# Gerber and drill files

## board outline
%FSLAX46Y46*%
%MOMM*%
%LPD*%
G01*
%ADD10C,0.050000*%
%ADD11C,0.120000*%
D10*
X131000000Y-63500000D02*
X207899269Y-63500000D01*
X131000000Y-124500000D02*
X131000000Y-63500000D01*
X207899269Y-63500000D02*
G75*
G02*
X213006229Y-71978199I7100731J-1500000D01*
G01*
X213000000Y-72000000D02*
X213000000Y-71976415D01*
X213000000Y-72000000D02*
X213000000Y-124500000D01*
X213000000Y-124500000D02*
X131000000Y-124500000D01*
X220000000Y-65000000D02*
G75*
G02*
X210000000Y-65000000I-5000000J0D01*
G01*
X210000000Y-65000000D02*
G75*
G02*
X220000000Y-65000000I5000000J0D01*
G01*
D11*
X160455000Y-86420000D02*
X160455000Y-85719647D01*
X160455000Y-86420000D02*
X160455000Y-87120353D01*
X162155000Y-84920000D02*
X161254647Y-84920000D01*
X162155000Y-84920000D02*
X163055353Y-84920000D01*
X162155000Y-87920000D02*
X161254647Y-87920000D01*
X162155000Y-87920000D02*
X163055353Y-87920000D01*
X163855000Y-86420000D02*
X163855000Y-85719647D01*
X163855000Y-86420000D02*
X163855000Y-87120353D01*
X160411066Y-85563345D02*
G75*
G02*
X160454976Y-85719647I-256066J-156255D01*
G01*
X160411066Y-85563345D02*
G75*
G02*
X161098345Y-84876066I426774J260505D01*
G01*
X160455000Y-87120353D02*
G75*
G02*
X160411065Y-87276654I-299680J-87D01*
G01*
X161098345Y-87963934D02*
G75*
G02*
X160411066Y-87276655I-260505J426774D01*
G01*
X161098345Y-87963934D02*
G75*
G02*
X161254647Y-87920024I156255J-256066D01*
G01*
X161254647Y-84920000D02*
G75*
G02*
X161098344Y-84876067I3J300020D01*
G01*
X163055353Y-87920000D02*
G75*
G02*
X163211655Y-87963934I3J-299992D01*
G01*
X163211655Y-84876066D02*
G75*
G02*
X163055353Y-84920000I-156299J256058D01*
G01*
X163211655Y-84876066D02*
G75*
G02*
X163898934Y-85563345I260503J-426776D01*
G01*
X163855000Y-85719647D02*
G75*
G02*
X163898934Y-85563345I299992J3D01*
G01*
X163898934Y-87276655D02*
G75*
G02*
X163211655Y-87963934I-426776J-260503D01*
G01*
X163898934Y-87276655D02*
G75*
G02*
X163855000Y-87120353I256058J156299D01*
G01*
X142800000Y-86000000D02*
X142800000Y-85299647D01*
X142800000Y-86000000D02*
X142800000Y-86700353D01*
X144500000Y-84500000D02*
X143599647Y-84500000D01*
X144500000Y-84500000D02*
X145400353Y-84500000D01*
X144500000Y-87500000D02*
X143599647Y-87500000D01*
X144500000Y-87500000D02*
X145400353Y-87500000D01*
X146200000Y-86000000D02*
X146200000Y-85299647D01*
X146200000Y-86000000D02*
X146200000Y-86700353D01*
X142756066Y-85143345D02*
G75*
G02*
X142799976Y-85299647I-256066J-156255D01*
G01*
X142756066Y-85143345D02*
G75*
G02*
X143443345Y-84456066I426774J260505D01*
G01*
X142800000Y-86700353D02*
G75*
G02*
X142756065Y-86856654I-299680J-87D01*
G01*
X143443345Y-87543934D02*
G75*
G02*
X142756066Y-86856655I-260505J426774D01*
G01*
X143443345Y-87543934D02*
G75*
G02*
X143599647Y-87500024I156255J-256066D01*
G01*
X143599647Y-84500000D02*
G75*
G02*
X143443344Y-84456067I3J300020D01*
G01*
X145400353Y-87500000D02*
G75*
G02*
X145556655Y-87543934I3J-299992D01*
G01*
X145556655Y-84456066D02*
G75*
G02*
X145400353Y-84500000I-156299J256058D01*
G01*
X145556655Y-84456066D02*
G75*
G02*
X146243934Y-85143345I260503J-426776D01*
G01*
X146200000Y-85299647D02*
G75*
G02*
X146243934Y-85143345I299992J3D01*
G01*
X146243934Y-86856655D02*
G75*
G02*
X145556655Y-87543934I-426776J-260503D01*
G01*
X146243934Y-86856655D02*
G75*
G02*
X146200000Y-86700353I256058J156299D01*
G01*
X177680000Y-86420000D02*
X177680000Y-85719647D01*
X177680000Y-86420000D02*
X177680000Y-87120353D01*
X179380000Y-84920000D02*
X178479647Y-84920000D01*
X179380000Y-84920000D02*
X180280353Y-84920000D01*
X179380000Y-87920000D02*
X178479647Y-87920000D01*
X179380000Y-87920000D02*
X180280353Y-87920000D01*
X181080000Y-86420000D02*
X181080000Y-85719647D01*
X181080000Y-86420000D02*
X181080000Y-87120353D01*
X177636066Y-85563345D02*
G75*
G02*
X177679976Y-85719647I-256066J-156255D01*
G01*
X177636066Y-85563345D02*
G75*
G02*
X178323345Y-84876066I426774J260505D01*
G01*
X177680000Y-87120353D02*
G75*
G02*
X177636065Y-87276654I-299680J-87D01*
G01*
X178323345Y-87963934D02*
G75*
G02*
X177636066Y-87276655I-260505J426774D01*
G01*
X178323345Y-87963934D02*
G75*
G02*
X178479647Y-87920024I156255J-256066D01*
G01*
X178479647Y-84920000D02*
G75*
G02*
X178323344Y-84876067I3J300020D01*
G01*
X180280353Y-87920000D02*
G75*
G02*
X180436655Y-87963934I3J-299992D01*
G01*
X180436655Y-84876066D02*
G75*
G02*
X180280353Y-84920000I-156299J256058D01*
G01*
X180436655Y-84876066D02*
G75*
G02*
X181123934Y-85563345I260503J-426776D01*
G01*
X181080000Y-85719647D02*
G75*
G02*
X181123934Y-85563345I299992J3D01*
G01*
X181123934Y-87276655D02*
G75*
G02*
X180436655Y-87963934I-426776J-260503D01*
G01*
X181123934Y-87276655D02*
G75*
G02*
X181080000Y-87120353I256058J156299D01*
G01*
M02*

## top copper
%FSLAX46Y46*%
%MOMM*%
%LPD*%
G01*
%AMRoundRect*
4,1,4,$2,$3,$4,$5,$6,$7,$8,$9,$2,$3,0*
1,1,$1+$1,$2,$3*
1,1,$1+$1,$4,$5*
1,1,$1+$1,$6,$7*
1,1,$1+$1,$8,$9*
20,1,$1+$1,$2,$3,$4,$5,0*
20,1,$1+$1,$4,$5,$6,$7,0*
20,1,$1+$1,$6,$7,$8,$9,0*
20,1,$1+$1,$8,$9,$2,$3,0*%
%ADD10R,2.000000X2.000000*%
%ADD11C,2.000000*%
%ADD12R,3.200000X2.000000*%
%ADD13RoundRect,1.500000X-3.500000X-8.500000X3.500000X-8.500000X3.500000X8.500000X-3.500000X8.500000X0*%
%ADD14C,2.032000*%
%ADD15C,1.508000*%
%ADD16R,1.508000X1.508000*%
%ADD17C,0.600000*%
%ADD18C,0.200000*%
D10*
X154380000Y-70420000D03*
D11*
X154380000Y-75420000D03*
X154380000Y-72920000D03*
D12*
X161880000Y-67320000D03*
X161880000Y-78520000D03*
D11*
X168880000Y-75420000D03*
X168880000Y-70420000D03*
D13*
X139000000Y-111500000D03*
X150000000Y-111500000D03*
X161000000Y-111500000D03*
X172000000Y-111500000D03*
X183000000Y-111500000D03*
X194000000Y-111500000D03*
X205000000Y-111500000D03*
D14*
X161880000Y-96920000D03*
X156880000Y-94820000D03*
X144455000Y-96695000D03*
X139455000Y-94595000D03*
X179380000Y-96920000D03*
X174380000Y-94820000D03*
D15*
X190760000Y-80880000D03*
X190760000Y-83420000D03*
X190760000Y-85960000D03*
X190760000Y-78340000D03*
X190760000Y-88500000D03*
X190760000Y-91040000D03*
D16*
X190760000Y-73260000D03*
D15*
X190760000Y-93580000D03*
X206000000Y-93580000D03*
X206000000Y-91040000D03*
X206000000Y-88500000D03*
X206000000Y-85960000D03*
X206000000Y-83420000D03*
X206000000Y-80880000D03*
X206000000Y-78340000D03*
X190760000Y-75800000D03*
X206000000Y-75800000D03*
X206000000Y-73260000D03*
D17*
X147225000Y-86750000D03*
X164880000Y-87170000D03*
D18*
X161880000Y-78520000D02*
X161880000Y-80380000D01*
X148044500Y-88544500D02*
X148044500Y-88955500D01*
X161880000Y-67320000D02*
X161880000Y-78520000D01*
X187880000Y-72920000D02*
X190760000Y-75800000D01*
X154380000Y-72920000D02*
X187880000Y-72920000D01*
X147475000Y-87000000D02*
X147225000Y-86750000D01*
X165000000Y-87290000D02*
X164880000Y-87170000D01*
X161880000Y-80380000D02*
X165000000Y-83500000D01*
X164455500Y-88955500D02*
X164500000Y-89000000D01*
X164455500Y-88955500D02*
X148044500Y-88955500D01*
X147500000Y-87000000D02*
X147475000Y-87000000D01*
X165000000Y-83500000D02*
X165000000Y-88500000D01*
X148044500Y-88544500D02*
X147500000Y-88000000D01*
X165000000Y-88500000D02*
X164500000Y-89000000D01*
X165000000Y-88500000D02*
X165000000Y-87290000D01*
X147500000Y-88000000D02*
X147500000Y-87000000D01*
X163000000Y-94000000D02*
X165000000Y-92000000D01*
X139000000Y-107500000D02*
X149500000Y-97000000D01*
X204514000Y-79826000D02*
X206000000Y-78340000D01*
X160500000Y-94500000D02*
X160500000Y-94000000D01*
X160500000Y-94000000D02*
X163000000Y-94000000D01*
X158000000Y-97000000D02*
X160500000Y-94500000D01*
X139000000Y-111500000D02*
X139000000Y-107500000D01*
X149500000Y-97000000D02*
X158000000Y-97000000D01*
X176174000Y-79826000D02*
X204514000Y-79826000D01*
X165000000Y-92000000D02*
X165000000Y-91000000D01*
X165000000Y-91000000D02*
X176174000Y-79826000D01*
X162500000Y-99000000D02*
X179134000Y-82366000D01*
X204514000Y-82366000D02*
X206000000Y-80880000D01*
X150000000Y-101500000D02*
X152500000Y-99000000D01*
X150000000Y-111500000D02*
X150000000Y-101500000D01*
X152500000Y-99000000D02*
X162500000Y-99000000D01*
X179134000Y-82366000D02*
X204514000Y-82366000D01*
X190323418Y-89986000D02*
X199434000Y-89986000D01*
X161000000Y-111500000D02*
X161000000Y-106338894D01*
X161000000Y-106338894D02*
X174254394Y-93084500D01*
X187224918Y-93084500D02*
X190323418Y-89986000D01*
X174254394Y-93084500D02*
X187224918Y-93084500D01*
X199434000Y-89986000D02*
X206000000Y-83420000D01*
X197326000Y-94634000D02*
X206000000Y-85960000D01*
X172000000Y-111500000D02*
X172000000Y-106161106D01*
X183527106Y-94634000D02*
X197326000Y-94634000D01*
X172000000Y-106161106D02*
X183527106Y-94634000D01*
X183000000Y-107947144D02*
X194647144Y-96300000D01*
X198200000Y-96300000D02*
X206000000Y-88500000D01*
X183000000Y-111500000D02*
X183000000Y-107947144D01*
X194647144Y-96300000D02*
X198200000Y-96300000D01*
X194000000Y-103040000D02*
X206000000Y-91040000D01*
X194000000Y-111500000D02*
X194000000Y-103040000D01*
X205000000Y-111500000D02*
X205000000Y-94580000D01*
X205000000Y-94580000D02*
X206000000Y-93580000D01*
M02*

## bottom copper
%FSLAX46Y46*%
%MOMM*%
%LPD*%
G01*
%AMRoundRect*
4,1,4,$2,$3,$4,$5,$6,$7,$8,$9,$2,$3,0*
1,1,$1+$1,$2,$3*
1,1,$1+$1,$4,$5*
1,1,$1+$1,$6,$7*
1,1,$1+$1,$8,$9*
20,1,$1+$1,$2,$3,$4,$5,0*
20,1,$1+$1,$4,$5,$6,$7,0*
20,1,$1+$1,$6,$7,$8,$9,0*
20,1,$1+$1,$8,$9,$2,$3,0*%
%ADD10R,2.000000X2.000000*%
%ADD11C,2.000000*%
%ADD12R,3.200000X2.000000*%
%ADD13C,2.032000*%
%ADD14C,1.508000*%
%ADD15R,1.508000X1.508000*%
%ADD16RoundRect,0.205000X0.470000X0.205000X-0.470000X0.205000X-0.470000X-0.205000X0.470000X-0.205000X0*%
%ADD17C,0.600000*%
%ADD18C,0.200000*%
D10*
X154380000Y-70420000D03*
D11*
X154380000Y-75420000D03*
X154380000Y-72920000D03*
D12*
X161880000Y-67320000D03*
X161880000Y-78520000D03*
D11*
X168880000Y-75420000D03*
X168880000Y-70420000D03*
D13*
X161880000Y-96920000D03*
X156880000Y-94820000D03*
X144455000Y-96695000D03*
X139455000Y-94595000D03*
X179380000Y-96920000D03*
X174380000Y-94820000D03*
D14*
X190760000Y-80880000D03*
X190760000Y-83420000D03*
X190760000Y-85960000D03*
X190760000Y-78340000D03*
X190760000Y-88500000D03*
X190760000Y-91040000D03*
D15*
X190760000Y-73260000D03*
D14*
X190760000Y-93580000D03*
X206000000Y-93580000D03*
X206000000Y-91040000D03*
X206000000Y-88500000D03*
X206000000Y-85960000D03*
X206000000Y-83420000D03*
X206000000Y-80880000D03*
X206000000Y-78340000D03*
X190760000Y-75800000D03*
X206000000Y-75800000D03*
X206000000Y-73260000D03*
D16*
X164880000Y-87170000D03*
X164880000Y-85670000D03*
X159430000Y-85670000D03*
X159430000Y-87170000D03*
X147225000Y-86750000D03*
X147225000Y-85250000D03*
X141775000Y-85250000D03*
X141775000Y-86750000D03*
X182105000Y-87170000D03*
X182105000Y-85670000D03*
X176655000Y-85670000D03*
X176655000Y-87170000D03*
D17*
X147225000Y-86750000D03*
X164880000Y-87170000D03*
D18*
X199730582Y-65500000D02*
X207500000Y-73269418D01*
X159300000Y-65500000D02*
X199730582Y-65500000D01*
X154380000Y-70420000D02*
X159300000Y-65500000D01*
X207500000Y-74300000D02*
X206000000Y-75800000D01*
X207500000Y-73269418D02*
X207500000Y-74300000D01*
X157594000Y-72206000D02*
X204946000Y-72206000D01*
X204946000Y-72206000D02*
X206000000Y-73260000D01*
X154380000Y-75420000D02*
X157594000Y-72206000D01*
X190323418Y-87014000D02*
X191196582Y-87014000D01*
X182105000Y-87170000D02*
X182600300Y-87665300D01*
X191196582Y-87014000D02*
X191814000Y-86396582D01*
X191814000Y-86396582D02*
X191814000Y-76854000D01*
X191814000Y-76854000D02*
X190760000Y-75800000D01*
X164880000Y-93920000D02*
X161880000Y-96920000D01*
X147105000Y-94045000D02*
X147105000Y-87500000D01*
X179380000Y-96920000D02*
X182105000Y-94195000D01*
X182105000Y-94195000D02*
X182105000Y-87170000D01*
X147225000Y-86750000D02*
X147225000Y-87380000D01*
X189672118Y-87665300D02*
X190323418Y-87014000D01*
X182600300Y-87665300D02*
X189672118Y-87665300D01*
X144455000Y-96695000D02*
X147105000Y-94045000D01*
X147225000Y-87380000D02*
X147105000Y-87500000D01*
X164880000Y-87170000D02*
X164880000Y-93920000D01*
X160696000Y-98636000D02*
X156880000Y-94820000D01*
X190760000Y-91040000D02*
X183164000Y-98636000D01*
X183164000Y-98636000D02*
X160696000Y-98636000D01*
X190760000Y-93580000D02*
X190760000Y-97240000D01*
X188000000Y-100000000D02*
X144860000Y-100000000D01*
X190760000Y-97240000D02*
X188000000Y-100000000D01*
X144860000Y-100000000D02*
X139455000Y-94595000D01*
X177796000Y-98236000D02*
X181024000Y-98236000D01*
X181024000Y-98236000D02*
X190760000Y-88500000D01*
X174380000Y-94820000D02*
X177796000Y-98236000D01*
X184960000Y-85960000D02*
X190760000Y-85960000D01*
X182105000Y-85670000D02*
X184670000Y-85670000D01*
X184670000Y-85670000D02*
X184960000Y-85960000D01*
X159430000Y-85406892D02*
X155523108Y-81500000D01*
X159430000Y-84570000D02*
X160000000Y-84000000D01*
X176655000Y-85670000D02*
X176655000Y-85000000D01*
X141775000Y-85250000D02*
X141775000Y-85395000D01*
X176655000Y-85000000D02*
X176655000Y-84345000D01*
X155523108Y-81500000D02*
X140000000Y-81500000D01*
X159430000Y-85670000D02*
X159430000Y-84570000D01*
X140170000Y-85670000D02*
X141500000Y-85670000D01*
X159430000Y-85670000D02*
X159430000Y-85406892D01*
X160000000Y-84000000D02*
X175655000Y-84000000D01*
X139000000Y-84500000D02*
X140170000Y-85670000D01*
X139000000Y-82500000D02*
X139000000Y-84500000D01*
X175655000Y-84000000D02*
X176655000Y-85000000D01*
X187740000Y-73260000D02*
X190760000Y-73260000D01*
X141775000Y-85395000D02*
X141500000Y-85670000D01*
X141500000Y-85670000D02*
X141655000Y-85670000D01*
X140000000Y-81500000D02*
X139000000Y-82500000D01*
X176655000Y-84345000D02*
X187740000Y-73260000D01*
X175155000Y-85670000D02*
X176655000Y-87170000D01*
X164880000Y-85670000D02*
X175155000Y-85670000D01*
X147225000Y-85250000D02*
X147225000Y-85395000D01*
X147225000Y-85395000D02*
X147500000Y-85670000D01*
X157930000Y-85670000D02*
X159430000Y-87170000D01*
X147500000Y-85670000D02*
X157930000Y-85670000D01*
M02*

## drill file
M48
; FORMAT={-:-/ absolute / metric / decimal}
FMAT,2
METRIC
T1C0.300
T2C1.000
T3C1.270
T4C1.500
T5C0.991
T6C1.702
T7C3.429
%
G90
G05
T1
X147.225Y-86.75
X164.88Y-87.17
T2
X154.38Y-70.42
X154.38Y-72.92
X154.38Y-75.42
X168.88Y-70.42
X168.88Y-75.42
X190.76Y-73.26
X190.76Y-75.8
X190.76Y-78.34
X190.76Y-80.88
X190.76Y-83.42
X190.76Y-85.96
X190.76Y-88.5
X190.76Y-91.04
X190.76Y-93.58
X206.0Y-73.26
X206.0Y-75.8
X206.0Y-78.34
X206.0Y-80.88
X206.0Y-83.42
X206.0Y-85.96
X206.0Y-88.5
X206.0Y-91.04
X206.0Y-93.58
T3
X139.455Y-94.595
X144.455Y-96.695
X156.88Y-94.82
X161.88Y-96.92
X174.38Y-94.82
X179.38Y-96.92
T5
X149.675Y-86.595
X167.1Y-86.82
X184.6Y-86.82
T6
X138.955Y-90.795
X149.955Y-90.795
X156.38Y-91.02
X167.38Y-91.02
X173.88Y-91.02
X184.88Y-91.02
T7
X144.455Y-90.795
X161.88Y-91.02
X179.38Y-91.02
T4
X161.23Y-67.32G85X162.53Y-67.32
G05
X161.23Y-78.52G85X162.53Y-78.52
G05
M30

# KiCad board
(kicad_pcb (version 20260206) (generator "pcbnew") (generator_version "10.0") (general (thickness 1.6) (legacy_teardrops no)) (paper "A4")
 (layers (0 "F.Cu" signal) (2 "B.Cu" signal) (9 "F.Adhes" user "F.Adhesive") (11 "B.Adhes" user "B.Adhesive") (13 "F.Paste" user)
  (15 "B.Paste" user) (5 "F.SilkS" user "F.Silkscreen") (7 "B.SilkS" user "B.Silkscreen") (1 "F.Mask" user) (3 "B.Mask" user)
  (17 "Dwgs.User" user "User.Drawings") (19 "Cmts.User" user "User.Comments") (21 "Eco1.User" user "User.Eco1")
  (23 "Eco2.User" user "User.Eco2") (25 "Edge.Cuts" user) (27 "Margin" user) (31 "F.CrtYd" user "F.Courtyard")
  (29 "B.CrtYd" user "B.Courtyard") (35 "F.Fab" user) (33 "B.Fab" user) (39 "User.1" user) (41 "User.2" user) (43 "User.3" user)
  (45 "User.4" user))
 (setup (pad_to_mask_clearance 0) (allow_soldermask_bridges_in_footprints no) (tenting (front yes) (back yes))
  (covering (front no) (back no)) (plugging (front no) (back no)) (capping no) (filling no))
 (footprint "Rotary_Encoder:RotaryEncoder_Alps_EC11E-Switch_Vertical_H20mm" (layer "F.Cu") (at 154.38 70.42)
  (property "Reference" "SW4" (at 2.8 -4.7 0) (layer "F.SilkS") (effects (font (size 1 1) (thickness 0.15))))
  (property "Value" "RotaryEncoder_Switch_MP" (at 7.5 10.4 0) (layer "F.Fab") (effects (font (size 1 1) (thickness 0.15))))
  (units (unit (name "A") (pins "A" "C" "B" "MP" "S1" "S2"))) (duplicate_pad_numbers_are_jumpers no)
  (pad "A" thru_hole rect (at 0 0) (size 2 2) (drill 1) (layers "*.Cu" "*.Mask") (remove_unused_layers no) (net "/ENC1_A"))
  (pad "B" thru_hole circle (at 0 5) (size 2 2) (drill 1) (layers "*.Cu" "*.Mask") (remove_unused_layers no) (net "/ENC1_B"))
  (pad "C" thru_hole circle (at 0 2.5) (size 2 2) (drill 1) (layers "*.Cu" "*.Mask") (remove_unused_layers no) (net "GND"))
  (pad "MP" thru_hole rect (at 7.5 -3.1) (size 3.2 2) (drill oval 2.8 1.5) (layers "*.Cu" "*.Mask") (remove_unused_layers no) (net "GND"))
  (pad "MP" thru_hole rect (at 7.5 8.1) (size 3.2 2) (drill oval 2.8 1.5) (layers "*.Cu" "*.Mask") (remove_unused_layers no) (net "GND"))
  (pad "S1" thru_hole circle (at 14.5 5) (size 2 2) (drill 1) (layers "*.Cu" "*.Mask") (remove_unused_layers no)
   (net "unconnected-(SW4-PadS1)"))
  (pad "S2" thru_hole circle (at 14.5 0) (size 2 2) (drill 1) (layers "*.Cu" "*.Mask") (remove_unused_layers no)
   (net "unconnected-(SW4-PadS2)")))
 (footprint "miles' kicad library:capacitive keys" (layer "F.Cu") (at 169 93.5)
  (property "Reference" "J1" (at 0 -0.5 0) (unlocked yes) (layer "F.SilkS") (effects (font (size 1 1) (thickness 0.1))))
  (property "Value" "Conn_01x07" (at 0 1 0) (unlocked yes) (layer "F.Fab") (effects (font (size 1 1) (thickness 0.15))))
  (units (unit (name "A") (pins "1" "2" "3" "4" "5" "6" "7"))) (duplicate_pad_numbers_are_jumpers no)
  (pad "1" smd roundrect (at -30 18) (size 10 20) (layers "F.Cu" "F.Mask") (roundrect_rratio 0.15) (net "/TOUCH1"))
  (pad "2" smd roundrect (at -19 18) (size 10 20) (layers "F.Cu" "F.Mask") (roundrect_rratio 0.15) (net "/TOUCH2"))
  (pad "3" smd roundrect (at -8 18) (size 10 20) (layers "F.Cu" "F.Mask") (roundrect_rratio 0.15) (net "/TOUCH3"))
  (pad "4" smd roundrect (at 3 18) (size 10 20) (layers "F.Cu" "F.Mask") (roundrect_rratio 0.15) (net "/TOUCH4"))
  (pad "5" smd roundrect (at 14 18) (size 10 20) (layers "F.Cu" "F.Mask") (roundrect_rratio 0.15) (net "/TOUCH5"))
  (pad "6" smd roundrect (at 25 18) (size 10 20) (layers "F.Cu" "F.Mask") (roundrect_rratio 0.15) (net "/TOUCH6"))
  (pad "7" smd roundrect (at 36 18) (size 10 20) (layers "F.Cu" "F.Mask") (roundrect_rratio 0.15) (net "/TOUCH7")))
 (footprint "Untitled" (layer "F.Cu") (at 163 40.5)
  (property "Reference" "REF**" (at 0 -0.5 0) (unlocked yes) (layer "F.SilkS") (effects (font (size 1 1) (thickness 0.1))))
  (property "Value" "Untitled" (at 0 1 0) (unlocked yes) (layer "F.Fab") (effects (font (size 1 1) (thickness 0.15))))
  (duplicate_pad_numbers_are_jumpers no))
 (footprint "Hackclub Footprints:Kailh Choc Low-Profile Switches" (layer "F.Cu") (at 161.88 91.02)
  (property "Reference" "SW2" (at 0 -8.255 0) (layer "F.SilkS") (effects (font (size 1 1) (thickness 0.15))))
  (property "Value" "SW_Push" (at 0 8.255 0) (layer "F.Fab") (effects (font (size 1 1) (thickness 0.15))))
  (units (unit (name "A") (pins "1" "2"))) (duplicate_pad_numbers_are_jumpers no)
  (pad "" np_thru_hole circle (at -5.5 0) (size 1.7018 1.7018) (drill 1.7018) (layers "*.Cu" "*.Mask"))
  (pad "" np_thru_hole circle (at 0 0) (size 3.429 3.429) (drill 3.429) (layers "*.Cu" "*.Mask"))
  (pad "" np_thru_hole circle (at 5.22 -4.2) (size 0.9906 0.9906) (drill 0.9906) (layers "*.Cu" "*.Mask"))
  (pad "" np_thru_hole circle (at 5.5 0) (size 1.7018 1.7018) (drill 1.7018) (layers "*.Cu" "*.Mask"))
  (pad "1" thru_hole circle (at 0 5.9) (size 2.032 2.032) (drill 1.27) (layers "*.Cu" "*.Mask") (remove_unused_layers no) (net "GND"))
  (pad "2" thru_hole circle (at -5 3.8) (size 2.032 2.032) (drill 1.27) (layers "*.Cu" "*.Mask") (remove_unused_layers no) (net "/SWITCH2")))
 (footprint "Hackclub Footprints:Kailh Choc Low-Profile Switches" (layer "F.Cu") (at 144.455 90.795)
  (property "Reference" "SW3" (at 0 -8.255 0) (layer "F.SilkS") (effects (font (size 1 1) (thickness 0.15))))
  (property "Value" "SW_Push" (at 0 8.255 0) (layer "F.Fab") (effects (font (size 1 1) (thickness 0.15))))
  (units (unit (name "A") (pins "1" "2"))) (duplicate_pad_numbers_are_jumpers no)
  (pad "" np_thru_hole circle (at -5.5 0) (size 1.7018 1.7018) (drill 1.7018) (layers "*.Cu" "*.Mask"))
  (pad "" np_thru_hole circle (at 0 0) (size 3.429 3.429) (drill 3.429) (layers "*.Cu" "*.Mask"))
  (pad "" np_thru_hole circle (at 5.22 -4.2) (size 0.9906 0.9906) (drill 0.9906) (layers "*.Cu" "*.Mask"))
  (pad "" np_thru_hole circle (at 5.5 0) (size 1.7018 1.7018) (drill 1.7018) (layers "*.Cu" "*.Mask"))
  (pad "1" thru_hole circle (at 0 5.9) (size 2.032 2.032) (drill 1.27) (layers "*.Cu" "*.Mask") (remove_unused_layers no) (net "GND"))
  (pad "2" thru_hole circle (at -5 3.8) (size 2.032 2.032) (drill 1.27) (layers "*.Cu" "*.Mask") (remove_unused_layers no) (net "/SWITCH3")))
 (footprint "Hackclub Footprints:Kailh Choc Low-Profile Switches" (layer "F.Cu") (at 179.38 91.02)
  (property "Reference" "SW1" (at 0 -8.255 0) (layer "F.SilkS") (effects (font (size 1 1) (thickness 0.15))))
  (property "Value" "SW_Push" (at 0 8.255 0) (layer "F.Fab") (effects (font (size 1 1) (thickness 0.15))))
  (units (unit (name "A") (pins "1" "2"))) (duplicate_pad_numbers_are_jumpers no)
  (pad "" np_thru_hole circle (at -5.5 0) (size 1.7018 1.7018) (drill 1.7018) (layers "*.Cu" "*.Mask"))
  (pad "" np_thru_hole circle (at 0 0) (size 3.429 3.429) (drill 3.429) (layers "*.Cu" "*.Mask"))
  (pad "" np_thru_hole circle (at 5.22 -4.2) (size 0.9906 0.9906) (drill 0.9906) (layers "*.Cu" "*.Mask"))
  (pad "" np_thru_hole circle (at 5.5 0) (size 1.7018 1.7018) (drill 1.7018) (layers "*.Cu" "*.Mask"))
  (pad "1" thru_hole circle (at 0 5.9) (size 2.032 2.032) (drill 1.27) (layers "*.Cu" "*.Mask") (remove_unused_layers no) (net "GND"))
  (pad "2" thru_hole circle (at -5 3.8) (size 2.032 2.032) (drill 1.27) (layers "*.Cu" "*.Mask") (remove_unused_layers no) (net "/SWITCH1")))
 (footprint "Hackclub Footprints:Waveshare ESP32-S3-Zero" (layer "F.Cu") (at 198.38 83.42)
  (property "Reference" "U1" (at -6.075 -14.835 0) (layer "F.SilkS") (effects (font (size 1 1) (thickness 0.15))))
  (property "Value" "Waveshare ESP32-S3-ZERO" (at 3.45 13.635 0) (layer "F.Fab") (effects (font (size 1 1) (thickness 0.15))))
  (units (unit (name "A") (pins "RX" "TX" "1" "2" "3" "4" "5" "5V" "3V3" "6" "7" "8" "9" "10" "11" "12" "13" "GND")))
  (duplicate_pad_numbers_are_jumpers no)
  (pad "1" thru_hole circle (at -7.62 -2.54) (size 1.508 1.508) (drill 1) (layers "*.Cu" "*.Mask") (remove_unused_layers no)
   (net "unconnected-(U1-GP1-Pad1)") (solder_mask_margin 0.102))
  (pad "2" thru_hole circle (at -7.62 0) (size 1.508 1.508) (drill 1) (layers "*.Cu" "*.Mask") (remove_unused_layers no)
   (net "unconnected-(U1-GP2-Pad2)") (solder_mask_margin 0.102))
  (pad "3" thru_hole circle (at -7.62 2.54) (size 1.508 1.508) (drill 1) (layers "*.Cu" "*.Mask") (remove_unused_layers no) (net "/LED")
   (solder_mask_margin 0.102))
  (pad "3V3" thru_hole circle (at -7.62 -5.08) (size 1.508 1.508) (drill 1) (layers "*.Cu" "*.Mask") (remove_unused_layers no) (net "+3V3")
   (solder_mask_margin 0.102))
  (pad "4" thru_hole circle (at -7.62 5.08) (size 1.508 1.508) (drill 1) (layers "*.Cu" "*.Mask") (remove_unused_layers no) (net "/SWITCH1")
   (solder_mask_margin 0.102))
  (pad "5" thru_hole circle (at -7.62 7.62) (size 1.508 1.508) (drill 1) (layers "*.Cu" "*.Mask") (remove_unused_layers no) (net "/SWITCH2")
   (solder_mask_margin 0.102))
  (pad "5V" thru_hole rect (at -7.62 -10.16) (size 1.508 1.508) (drill 1) (layers "*.Cu" "*.Mask") (remove_unused_layers no) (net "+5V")
   (solder_mask_margin 0.102))
  (pad "6" thru_hole circle (at -7.62 10.16) (size 1.508 1.508) (drill 1) (layers "*.Cu" "*.Mask") (remove_unused_layers no)
   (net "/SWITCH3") (solder_mask_margin 0.102))
  (pad "7" thru_hole circle (at 7.62 10.16) (size 1.508 1.508) (drill 1) (layers "*.Cu" "*.Mask") (remove_unused_layers no) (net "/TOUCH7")
   (solder_mask_margin 0.102))
  (pad "8" thru_hole circle (at 7.62 7.62) (size 1.508 1.508) (drill 1) (layers "*.Cu" "*.Mask") (remove_unused_layers no) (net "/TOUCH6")
   (solder_mask_margin 0.102))
  (pad "9" thru_hole circle (at 7.62 5.08) (size 1.508 1.508) (drill 1) (layers "*.Cu" "*.Mask") (remove_unused_layers no) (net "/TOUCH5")
   (solder_mask_margin 0.102))
  (pad "10" thru_hole circle (at 7.62 2.54) (size 1.508 1.508) (drill 1) (layers "*.Cu" "*.Mask") (remove_unused_layers no) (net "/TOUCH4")
   (solder_mask_margin 0.102))
  (pad "11" thru_hole circle (at 7.62 0) (size 1.508 1.508) (drill 1) (layers "*.Cu" "*.Mask") (remove_unused_layers no) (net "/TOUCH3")
   (solder_mask_margin 0.102))
  (pad "12" thru_hole circle (at 7.62 -2.54) (size 1.508 1.508) (drill 1) (layers "*.Cu" "*.Mask") (remove_unused_layers no) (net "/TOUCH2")
   (solder_mask_margin 0.102))
  (pad "13" thru_hole circle (at 7.62 -5.08) (size 1.508 1.508) (drill 1) (layers "*.Cu" "*.Mask") (remove_unused_layers no) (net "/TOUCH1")
   (solder_mask_margin 0.102))
  (pad "GND" thru_hole circle (at -7.62 -7.62) (size 1.508 1.508) (drill 1) (layers "*.Cu" "*.Mask") (remove_unused_layers no) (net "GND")
   (solder_mask_margin 0.102))
  (pad "RX" thru_hole circle (at 7.62 -7.62) (size 1.508 1.508) (drill 1) (layers "*.Cu" "*.Mask") (remove_unused_layers no) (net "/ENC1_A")
   (solder_mask_margin 0.102))
  (pad "TX" thru_hole circle (at 7.62 -10.16) (size 1.508 1.508) (drill 1) (layers "*.Cu" "*.Mask") (remove_unused_layers no)
   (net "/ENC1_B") (solder_mask_margin 0.102)))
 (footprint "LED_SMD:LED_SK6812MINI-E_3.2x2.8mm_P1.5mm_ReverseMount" (layer "B.Cu") (at 162.155 86.42 180)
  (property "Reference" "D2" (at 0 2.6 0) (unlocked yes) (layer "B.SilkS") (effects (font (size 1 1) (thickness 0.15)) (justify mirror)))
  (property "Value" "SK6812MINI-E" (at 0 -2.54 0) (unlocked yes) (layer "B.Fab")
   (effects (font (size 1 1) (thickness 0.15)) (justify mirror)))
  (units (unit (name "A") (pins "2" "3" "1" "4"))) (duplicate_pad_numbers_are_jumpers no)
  (fp_line (start 1.7 0) (end 1.7 0.700353) (stroke (width 0.12) (type solid)) (layer "Edge.Cuts"))
  (fp_line (start 1.7 0) (end 1.7 -0.700353) (stroke (width 0.12) (type solid)) (layer "Edge.Cuts"))
  (fp_line (start 0 1.5) (end 0.900353 1.5) (stroke (width 0.12) (type solid)) (layer "Edge.Cuts"))
  (fp_line (start 0 1.5) (end -0.900353 1.5) (stroke (width 0.12) (type solid)) (layer "Edge.Cuts"))
  (fp_line (start 0 -1.5) (end 0.900353 -1.5) (stroke (width 0.12) (type solid)) (layer "Edge.Cuts"))
  (fp_line (start 0 -1.5) (end -0.900353 -1.5) (stroke (width 0.12) (type solid)) (layer "Edge.Cuts"))
  (fp_line (start -1.7 0) (end -1.7 0.700353) (stroke (width 0.12) (type solid)) (layer "Edge.Cuts"))
  (fp_line (start -1.7 0) (end -1.7 -0.700353) (stroke (width 0.12) (type solid)) (layer "Edge.Cuts"))
  (fp_arc (start 1.743934 0.856655) (mid 1.711191 0.781533) (end 1.7 0.700353) (stroke (width 0.12) (type solid)) (layer "Edge.Cuts"))
  (fp_arc (start 1.743934 0.856655) (mid 1.670713 1.470713) (end 1.056655 1.543934) (stroke (width 0.12) (type solid)) (layer "Edge.Cuts"))
  (fp_arc (start 1.7 -0.700353) (mid 1.711181 -0.781538) (end 1.743934 -0.856655) (stroke (width 0.12) (type solid)) (layer "Edge.Cuts"))
  (fp_arc (start 1.056655 -1.543934) (mid 1.670711 -1.470711) (end 1.743934 -0.856655) (stroke (width 0.12) (type solid))
   (layer "Edge.Cuts"))
  (fp_arc (start 1.056655 -1.543934) (mid 0.981533 -1.511191) (end 0.900353 -1.5) (stroke (width 0.12) (type solid)) (layer "Edge.Cuts"))
  (fp_arc (start 0.900353 1.5) (mid 0.981532 1.511193) (end 1.056655 1.543934) (stroke (width 0.12) (type solid)) (layer "Edge.Cuts"))
  (fp_arc (start -0.900353 -1.5) (mid -0.981533 -1.511192) (end -1.056655 -1.543934) (stroke (width 0.12) (type solid)) (layer "Edge.Cuts"))
  (fp_arc (start -1.056655 1.543934) (mid -0.981533 1.511192) (end -0.900353 1.5) (stroke (width 0.12) (type solid)) (layer "Edge.Cuts"))
  (fp_arc (start -1.056655 1.543934) (mid -1.670711 1.470711) (end -1.743934 0.856655) (stroke (width 0.12) (type solid))
   (layer "Edge.Cuts"))
  (fp_arc (start -1.7 0.700353) (mid -1.711192 0.781533) (end -1.743934 0.856655) (stroke (width 0.12) (type solid)) (layer "Edge.Cuts"))
  (fp_arc (start -1.743934 -0.856655) (mid -1.670711 -1.470711) (end -1.056655 -1.543934) (stroke (width 0.12) (type solid))
   (layer "Edge.Cuts"))
  (fp_arc (start -1.743934 -0.856655) (mid -1.711192 -0.781533) (end -1.7 -0.700353) (stroke (width 0.12) (type solid)) (layer "Edge.Cuts"))
  (pad "1" smd roundrect (at -2.725 -0.75 180) (size 1.35 0.82) (layers "B.Cu" "B.Mask" "B.Paste") (roundrect_rratio 0.25) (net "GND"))
  (pad "2" smd roundrect (at -2.725 0.75 180) (size 1.35 0.82) (layers "B.Cu" "B.Mask" "B.Paste") (roundrect_rratio 0.25)
   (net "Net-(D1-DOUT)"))
  (pad "3" smd roundrect (at 2.725 0.75 180) (size 1.35 0.82) (layers "B.Cu" "B.Mask" "B.Paste") (roundrect_rratio 0.25) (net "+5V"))
  (pad "4" smd roundrect (at 2.725 -0.75 180) (size 1.35 0.82) (layers "B.Cu" "B.Mask" "B.Paste") (roundrect_rratio 0.25)
   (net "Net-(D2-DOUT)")))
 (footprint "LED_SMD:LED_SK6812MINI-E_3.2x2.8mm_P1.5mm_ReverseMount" (layer "B.Cu") (at 144.5 86 180)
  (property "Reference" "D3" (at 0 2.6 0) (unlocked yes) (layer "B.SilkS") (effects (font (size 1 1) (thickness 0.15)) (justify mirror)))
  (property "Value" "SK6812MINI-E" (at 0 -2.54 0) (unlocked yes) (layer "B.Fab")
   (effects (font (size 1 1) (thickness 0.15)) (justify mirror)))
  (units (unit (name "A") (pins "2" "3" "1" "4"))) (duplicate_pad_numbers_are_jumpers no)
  (fp_line (start 1.7 0) (end 1.7 0.700353) (stroke (width 0.12) (type solid)) (layer "Edge.Cuts"))
  (fp_line (start 1.7 0) (end 1.7 -0.700353) (stroke (width 0.12) (type solid)) (layer "Edge.Cuts"))
  (fp_line (start 0 1.5) (end 0.900353 1.5) (stroke (width 0.12) (type solid)) (layer "Edge.Cuts"))
  (fp_line (start 0 1.5) (end -0.900353 1.5) (stroke (width 0.12) (type solid)) (layer "Edge.Cuts"))
  (fp_line (start 0 -1.5) (end 0.900353 -1.5) (stroke (width 0.12) (type solid)) (layer "Edge.Cuts"))
  (fp_line (start 0 -1.5) (end -0.900353 -1.5) (stroke (width 0.12) (type solid)) (layer "Edge.Cuts"))
  (fp_line (start -1.7 0) (end -1.7 0.700353) (stroke (width 0.12) (type solid)) (layer "Edge.Cuts"))
  (fp_line (start -1.7 0) (end -1.7 -0.700353) (stroke (width 0.12) (type solid)) (layer "Edge.Cuts"))
  (fp_arc (start 1.743934 0.856655) (mid 1.711191 0.781533) (end 1.7 0.700353) (stroke (width 0.12) (type solid)) (layer "Edge.Cuts"))
  (fp_arc (start 1.743934 0.856655) (mid 1.670713 1.470713) (end 1.056655 1.543934) (stroke (width 0.12) (type solid)) (layer "Edge.Cuts"))
  (fp_arc (start 1.7 -0.700353) (mid 1.711181 -0.781538) (end 1.743934 -0.856655) (stroke (width 0.12) (type solid)) (layer "Edge.Cuts"))
  (fp_arc (start 1.056655 -1.543934) (mid 1.670711 -1.470711) (end 1.743934 -0.856655) (stroke (width 0.12) (type solid))
   (layer "Edge.Cuts"))
  (fp_arc (start 1.056655 -1.543934) (mid 0.981533 -1.511191) (end 0.900353 -1.5) (stroke (width 0.12) (type solid)) (layer "Edge.Cuts"))
  (fp_arc (start 0.900353 1.5) (mid 0.981532 1.511193) (end 1.056655 1.543934) (stroke (width 0.12) (type solid)) (layer "Edge.Cuts"))
  (fp_arc (start -0.900353 -1.5) (mid -0.981533 -1.511192) (end -1.056655 -1.543934) (stroke (width 0.12) (type solid)) (layer "Edge.Cuts"))
  (fp_arc (start -1.056655 1.543934) (mid -0.981533 1.511192) (end -0.900353 1.5) (stroke (width 0.12) (type solid)) (layer "Edge.Cuts"))
  (fp_arc (start -1.056655 1.543934) (mid -1.670711 1.470711) (end -1.743934 0.856655) (stroke (width 0.12) (type solid))
   (layer "Edge.Cuts"))
  (fp_arc (start -1.7 0.700353) (mid -1.711192 0.781533) (end -1.743934 0.856655) (stroke (width 0.12) (type solid)) (layer "Edge.Cuts"))
  (fp_arc (start -1.743934 -0.856655) (mid -1.670711 -1.470711) (end -1.056655 -1.543934) (stroke (width 0.12) (type solid))
   (layer "Edge.Cuts"))
  (fp_arc (start -1.743934 -0.856655) (mid -1.711192 -0.781533) (end -1.7 -0.700353) (stroke (width 0.12) (type solid)) (layer "Edge.Cuts"))
  (pad "1" smd roundrect (at -2.725 -0.75 180) (size 1.35 0.82) (layers "B.Cu" "B.Mask" "B.Paste") (roundrect_rratio 0.25) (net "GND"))
  (pad "2" smd roundrect (at -2.725 0.75 180) (size 1.35 0.82) (layers "B.Cu" "B.Mask" "B.Paste") (roundrect_rratio 0.25)
   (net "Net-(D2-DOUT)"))
  (pad "3" smd roundrect (at 2.725 0.75 180) (size 1.35 0.82) (layers "B.Cu" "B.Mask" "B.Paste") (roundrect_rratio 0.25) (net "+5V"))
  (pad "4" smd roundrect (at 2.725 -0.75 180) (size 1.35 0.82) (layers "B.Cu" "B.Mask" "B.Paste") (roundrect_rratio 0.25)
   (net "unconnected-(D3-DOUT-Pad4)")))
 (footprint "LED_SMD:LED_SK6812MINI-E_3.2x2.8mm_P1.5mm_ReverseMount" (layer "B.Cu") (at 179.38 86.42 180)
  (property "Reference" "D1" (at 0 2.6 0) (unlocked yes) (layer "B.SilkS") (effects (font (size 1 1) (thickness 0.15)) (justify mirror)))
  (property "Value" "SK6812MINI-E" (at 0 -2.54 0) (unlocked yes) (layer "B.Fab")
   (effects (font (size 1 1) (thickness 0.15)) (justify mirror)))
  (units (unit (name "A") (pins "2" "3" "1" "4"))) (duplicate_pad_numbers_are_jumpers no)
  (fp_line (start 1.7 0) (end 1.7 0.700353) (stroke (width 0.12) (type solid)) (layer "Edge.Cuts"))
  (fp_line (start 1.7 0) (end 1.7 -0.700353) (stroke (width 0.12) (type solid)) (layer "Edge.Cuts"))
  (fp_line (start 0 1.5) (end 0.900353 1.5) (stroke (width 0.12) (type solid)) (layer "Edge.Cuts"))
  (fp_line (start 0 1.5) (end -0.900353 1.5) (stroke (width 0.12) (type solid)) (layer "Edge.Cuts"))
  (fp_line (start 0 -1.5) (end 0.900353 -1.5) (stroke (width 0.12) (type solid)) (layer "Edge.Cuts"))
  (fp_line (start 0 -1.5) (end -0.900353 -1.5) (stroke (width 0.12) (type solid)) (layer "Edge.Cuts"))
  (fp_line (start -1.7 0) (end -1.7 0.700353) (stroke (width 0.12) (type solid)) (layer "Edge.Cuts"))
  (fp_line (start -1.7 0) (end -1.7 -0.700353) (stroke (width 0.12) (type solid)) (layer "Edge.Cuts"))
  (fp_arc (start 1.743934 0.856655) (mid 1.711191 0.781533) (end 1.7 0.700353) (stroke (width 0.12) (type solid)) (layer "Edge.Cuts"))
  (fp_arc (start 1.743934 0.856655) (mid 1.670713 1.470713) (end 1.056655 1.543934) (stroke (width 0.12) (type solid)) (layer "Edge.Cuts"))
  (fp_arc (start 1.7 -0.700353) (mid 1.711181 -0.781538) (end 1.743934 -0.856655) (stroke (width 0.12) (type solid)) (layer "Edge.Cuts"))
  (fp_arc (start 1.056655 -1.543934) (mid 1.670711 -1.470711) (end 1.743934 -0.856655) (stroke (width 0.12) (type solid))
   (layer "Edge.Cuts"))
  (fp_arc (start 1.056655 -1.543934) (mid 0.981533 -1.511191) (end 0.900353 -1.5) (stroke (width 0.12) (type solid)) (layer "Edge.Cuts"))
  (fp_arc (start 0.900353 1.5) (mid 0.981532 1.511193) (end 1.056655 1.543934) (stroke (width 0.12) (type solid)) (layer "Edge.Cuts"))
  (fp_arc (start -0.900353 -1.5) (mid -0.981533 -1.511192) (end -1.056655 -1.543934) (stroke (width 0.12) (type solid)) (layer "Edge.Cuts"))
  (fp_arc (start -1.056655 1.543934) (mid -0.981533 1.511192) (end -0.900353 1.5) (stroke (width 0.12) (type solid)) (layer "Edge.Cuts"))
  (fp_arc (start -1.056655 1.543934) (mid -1.670711 1.470711) (end -1.743934 0.856655) (stroke (width 0.12) (type solid))
   (layer "Edge.Cuts"))
  (fp_arc (start -1.7 0.700353) (mid -1.711192 0.781533) (end -1.743934 0.856655) (stroke (width 0.12) (type solid)) (layer "Edge.Cuts"))
  (fp_arc (start -1.743934 -0.856655) (mid -1.670711 -1.470711) (end -1.056655 -1.543934) (stroke (width 0.12) (type solid))
   (layer "Edge.Cuts"))
  (fp_arc (start -1.743934 -0.856655) (mid -1.711192 -0.781533) (end -1.7 -0.700353) (stroke (width 0.12) (type solid)) (layer "Edge.Cuts"))
  (pad "1" smd roundrect (at -2.725 -0.75 180) (size 1.35 0.82) (layers "B.Cu" "B.Mask" "B.Paste") (roundrect_rratio 0.25) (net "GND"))
  (pad "2" smd roundrect (at -2.725 0.75 180) (size 1.35 0.82) (layers "B.Cu" "B.Mask" "B.Paste") (roundrect_rratio 0.25) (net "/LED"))
  (pad "3" smd roundrect (at 2.725 0.75 180) (size 1.35 0.82) (layers "B.Cu" "B.Mask" "B.Paste") (roundrect_rratio 0.25) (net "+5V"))
  (pad "4" smd roundrect (at 2.725 -0.75 180) (size 1.35 0.82) (layers "B.Cu" "B.Mask" "B.Paste") (roundrect_rratio 0.25)
   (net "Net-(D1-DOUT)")))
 (gr_line (start 131 63.5) (end 207.899269 63.5) (stroke (width 0.05) (type default)) (layer "Edge.Cuts"))
 (gr_line (start 131 124.5) (end 131 63.5) (stroke (width 0.05) (type default)) (layer "Edge.Cuts"))
 (gr_arc (start 207.899269 63.5) (mid 221.216708 61.25528) (end 213.006229 71.978199) (stroke (width 0.05) (type default))
  (layer "Edge.Cuts"))
 (gr_line (start 213 72) (end 213 71.976415) (stroke (width 0.05) (type default)) (layer "Edge.Cuts"))
 (gr_line (start 213 72) (end 213 124.5) (stroke (width 0.05) (type default)) (layer "Edge.Cuts"))
 (gr_line (start 213 124.5) (end 131 124.5) (stroke (width 0.05) (type default)) (layer "Edge.Cuts"))
 (gr_circle (center 215 65) (end 220 65) (stroke (width 0.05) (type default)) (fill no) (layer "Edge.Cuts"))
 (segment (start 199.730582 65.5) (end 207.5 73.269418) (width 0.2) (layer "B.Cu") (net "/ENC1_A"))
 (segment (start 159.3 65.5) (end 199.730582 65.5) (width 0.2) (layer "B.Cu") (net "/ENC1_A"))
 (segment (start 154.38 70.42) (end 159.3 65.5) (width 0.2) (layer "B.Cu") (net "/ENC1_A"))
 (segment (start 207.5 74.3) (end 206 75.8) (width 0.2) (layer "B.Cu") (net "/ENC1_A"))
 (segment (start 207.5 73.269418) (end 207.5 74.3) (width 0.2) (layer "B.Cu") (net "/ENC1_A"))
 (segment (start 157.594 72.206) (end 204.946 72.206) (width 0.2) (layer "B.Cu") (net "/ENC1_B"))
 (segment (start 204.946 72.206) (end 206 73.26) (width 0.2) (layer "B.Cu") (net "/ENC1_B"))
 (segment (start 154.38 75.42) (end 157.594 72.206) (width 0.2) (layer "B.Cu") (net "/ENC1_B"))
 (segment (start 161.88 78.52) (end 161.88 80.38) (width 0.2) (layer "F.Cu") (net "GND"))
 (segment (start 148.0445 88.5445) (end 148.0445 88.9555) (width 0.2) (layer "F.Cu") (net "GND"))
 (segment (start 161.88 67.32) (end 161.88 78.52) (width 0.2) (layer "F.Cu") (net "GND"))
 (segment (start 187.88 72.92) (end 190.76 75.8) (width 0.2) (layer "F.Cu") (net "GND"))
 (segment (start 154.38 72.92) (end 187.88 72.92) (width 0.2) (layer "F.Cu") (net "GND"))
 (segment (start 147.475 87) (end 147.225 86.75) (width 0.2) (layer "F.Cu") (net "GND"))
 (segment (start 165 87.29) (end 164.88 87.17) (width 0.2) (layer "F.Cu") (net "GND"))
 (segment (start 161.88 80.38) (end 165 83.5) (width 0.2) (layer "F.Cu") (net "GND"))
 (segment (start 164.4555 88.9555) (end 164.5 89) (width 0.2) (layer "F.Cu") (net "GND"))
 (segment (start 164.4555 88.9555) (end 148.0445 88.9555) (width 0.2) (layer "F.Cu") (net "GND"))
 (segment (start 147.5 87) (end 147.475 87) (width 0.2) (layer "F.Cu") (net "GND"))
 (segment (start 165 83.5) (end 165 88.5) (width 0.2) (layer "F.Cu") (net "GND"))
 (segment (start 148.0445 88.5445) (end 147.5 88) (width 0.2) (layer "F.Cu") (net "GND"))
 (segment (start 165 88.5) (end 164.5 89) (width 0.2) (layer "F.Cu") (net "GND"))
 (segment (start 165 88.5) (end 165 87.29) (width 0.2) (layer "F.Cu") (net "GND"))
 (segment (start 147.5 88) (end 147.5 87) (width 0.2) (layer "F.Cu") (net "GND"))
 (via (at 147.225 86.75) (size 0.6) (drill 0.3) (layers "F.Cu" "B.Cu") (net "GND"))
 (via (at 164.88 87.17) (size 0.6) (drill 0.3) (layers "F.Cu" "B.Cu") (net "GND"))
 (segment (start 190.323418 87.014) (end 191.196582 87.014) (width 0.2) (layer "B.Cu") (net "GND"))
 (segment (start 182.105 87.17) (end 182.6003 87.6653) (width 0.2) (layer "B.Cu") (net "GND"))
 (segment (start 191.196582 87.014) (end 191.814 86.396582) (width 0.2) (layer "B.Cu") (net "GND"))
 (segment (start 191.814 86.396582) (end 191.814 76.854) (width 0.2) (layer "B.Cu") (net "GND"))
 (segment (start 191.814 76.854) (end 190.76 75.8) (width 0.2) (layer "B.Cu") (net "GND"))
 (segment (start 164.88 93.92) (end 161.88 96.92) (width 0.2) (layer "B.Cu") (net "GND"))
 (segment (start 147.105 94.045) (end 147.105 87.5) (width 0.2) (layer "B.Cu") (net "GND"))
 (segment (start 179.38 96.92) (end 182.105 94.195) (width 0.2) (layer "B.Cu") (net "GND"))
 (segment (start 182.105 94.195) (end 182.105 87.17) (width 0.2) (layer "B.Cu") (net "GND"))
 (segment (start 147.225 86.75) (end 147.225 87.38) (width 0.2) (layer "B.Cu") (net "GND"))
 (segment (start 189.672118 87.6653) (end 190.323418 87.014) (width 0.2) (layer "B.Cu") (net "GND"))
 (segment (start 182.6003 87.6653) (end 189.672118 87.6653) (width 0.2) (layer "B.Cu") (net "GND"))
 (segment (start 144.455 96.695) (end 147.105 94.045) (width 0.2) (layer "B.Cu") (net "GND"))
 (segment (start 147.225 87.38) (end 147.105 87.5) (width 0.2) (layer "B.Cu") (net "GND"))
 (segment (start 164.88 87.17) (end 164.88 93.92) (width 0.2) (layer "B.Cu") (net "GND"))
 (segment (start 163 94) (end 165 92) (width 0.2) (layer "F.Cu") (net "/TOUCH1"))
 (segment (start 139 107.5) (end 149.5 97) (width 0.2) (layer "F.Cu") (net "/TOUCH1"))
 (segment (start 204.514 79.826) (end 206 78.34) (width 0.2) (layer "F.Cu") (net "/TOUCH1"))
 (segment (start 160.5 94.5) (end 160.5 94) (width 0.2) (layer "F.Cu") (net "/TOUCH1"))
 (segment (start 160.5 94) (end 163 94) (width 0.2) (layer "F.Cu") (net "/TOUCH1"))
 (segment (start 158 97) (end 160.5 94.5) (width 0.2) (layer "F.Cu") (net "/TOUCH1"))
 (segment (start 139 111.5) (end 139 107.5) (width 0.2) (layer "F.Cu") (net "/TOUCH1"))
 (segment (start 149.5 97) (end 158 97) (width 0.2) (layer "F.Cu") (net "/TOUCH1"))
 (segment (start 176.174 79.826) (end 204.514 79.826) (width 0.2) (layer "F.Cu") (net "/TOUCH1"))
 (segment (start 165 92) (end 165 91) (width 0.2) (layer "F.Cu") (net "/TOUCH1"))
 (segment (start 165 91) (end 176.174 79.826) (width 0.2) (layer "F.Cu") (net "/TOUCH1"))
 (segment (start 162.5 99) (end 179.134 82.366) (width 0.2) (layer "F.Cu") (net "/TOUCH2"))
 (segment (start 204.514 82.366) (end 206 80.88) (width 0.2) (layer "F.Cu") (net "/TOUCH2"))
 (segment (start 150 101.5) (end 152.5 99) (width 0.2) (layer "F.Cu") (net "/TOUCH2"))
 (segment (start 150 111.5) (end 150 101.5) (width 0.2) (layer "F.Cu") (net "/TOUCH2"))
 (segment (start 152.5 99) (end 162.5 99) (width 0.2) (layer "F.Cu") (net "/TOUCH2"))
 (segment (start 179.134 82.366) (end 204.514 82.366) (width 0.2) (layer "F.Cu") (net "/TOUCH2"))
 (segment (start 190.323418 89.986) (end 199.434 89.986) (width 0.2) (layer "F.Cu") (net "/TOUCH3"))
 (segment (start 161 111.5) (end 161 106.338894) (width 0.2) (layer "F.Cu") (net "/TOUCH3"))
 (segment (start 161 106.338894) (end 174.254394 93.0845) (width 0.2) (layer "F.Cu") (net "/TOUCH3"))
 (segment (start 187.224918 93.0845) (end 190.323418 89.986) (width 0.2) (layer "F.Cu") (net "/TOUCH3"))
 (segment (start 174.254394 93.0845) (end 187.224918 93.0845) (width 0.2) (layer "F.Cu") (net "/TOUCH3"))
 (segment (start 199.434 89.986) (end 206 83.42) (width 0.2) (layer "F.Cu") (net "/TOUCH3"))
 (segment (start 197.326 94.634) (end 206 85.96) (width 0.2) (layer "F.Cu") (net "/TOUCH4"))
 (segment (start 172 111.5) (end 172 106.161106) (width 0.2) (layer "F.Cu") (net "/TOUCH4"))
 (segment (start 183.527106 94.634) (end 197.326 94.634) (width 0.2) (layer "F.Cu") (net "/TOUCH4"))
 (segment (start 172 106.161106) (end 183.527106 94.634) (width 0.2) (layer "F.Cu") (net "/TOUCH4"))
 (segment (start 183 107.947144) (end 194.647144 96.3) (width 0.2) (layer "F.Cu") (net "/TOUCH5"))
 (segment (start 198.2 96.3) (end 206 88.5) (width 0.2) (layer "F.Cu") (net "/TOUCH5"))
 (segment (start 183 111.5) (end 183 107.947144) (width 0.2) (layer "F.Cu") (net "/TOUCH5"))
 (segment (start 194.647144 96.3) (end 198.2 96.3) (width 0.2) (layer "F.Cu") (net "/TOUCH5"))
 (segment (start 194 103.04) (end 206 91.04) (width 0.2) (layer "F.Cu") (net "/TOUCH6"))
 (segment (start 194 111.5) (end 194 103.04) (width 0.2) (layer "F.Cu") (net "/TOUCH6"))
 (segment (start 205 111.5) (end 205 94.58) (width 0.2) (layer "F.Cu") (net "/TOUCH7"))
 (segment (start 205 94.58) (end 206 93.58) (width 0.2) (layer "F.Cu") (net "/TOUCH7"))
 (segment (start 160.696 98.636) (end 156.88 94.82) (width 0.2) (layer "B.Cu") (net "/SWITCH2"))
 (segment (start 190.76 91.04) (end 183.164 98.636) (width 0.2) (layer "B.Cu") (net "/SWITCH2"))
 (segment (start 183.164 98.636) (end 160.696 98.636) (width 0.2) (layer "B.Cu") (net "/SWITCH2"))
 (segment (start 190.76 93.58) (end 190.76 97.24) (width 0.2) (layer "B.Cu") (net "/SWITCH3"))
 (segment (start 188 100) (end 144.86 100) (width 0.2) (layer "B.Cu") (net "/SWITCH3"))
 (segment (start 190.76 97.24) (end 188 100) (width 0.2) (layer "B.Cu") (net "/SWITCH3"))
 (segment (start 144.86 100) (end 139.455 94.595) (width 0.2) (layer "B.Cu") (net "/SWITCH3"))
 (segment (start 177.796 98.236) (end 181.024 98.236) (width 0.2) (layer "B.Cu") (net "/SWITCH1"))
 (segment (start 181.024 98.236) (end 190.76 88.5) (width 0.2) (layer "B.Cu") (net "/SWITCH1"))
 (segment (start 174.38 94.82) (end 177.796 98.236) (width 0.2) (layer "B.Cu") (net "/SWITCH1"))
 (segment (start 184.96 85.96) (end 190.76 85.96) (width 0.2) (layer "B.Cu") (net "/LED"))
 (segment (start 182.105 85.67) (end 184.67 85.67) (width 0.2) (layer "B.Cu") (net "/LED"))
 (segment (start 184.67 85.67) (end 184.96 85.96) (width 0.2) (layer "B.Cu") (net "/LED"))
 (segment (start 159.43 85.406892) (end 155.523108 81.5) (width 0.2) (layer "B.Cu") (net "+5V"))
 (segment (start 159.43 84.57) (end 160 84) (width 0.2) (layer "B.Cu") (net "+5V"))
 (segment (start 176.655 85.67) (end 176.655 85) (width 0.2) (layer "B.Cu") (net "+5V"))
 (segment (start 141.775 85.25) (end 141.775 85.395) (width 0.2) (layer "B.Cu") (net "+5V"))
 (segment (start 176.655 85) (end 176.655 84.345) (width 0.2) (layer "B.Cu") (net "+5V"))
 (segment (start 155.523108 81.5) (end 140 81.5) (width 0.2) (layer "B.Cu") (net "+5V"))
 (segment (start 159.43 85.67) (end 159.43 84.57) (width 0.2) (layer "B.Cu") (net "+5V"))
 (segment (start 140.17 85.67) (end 141.5 85.67) (width 0.2) (layer "B.Cu") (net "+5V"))
 (segment (start 159.43 85.67) (end 159.43 85.406892) (width 0.2) (layer "B.Cu") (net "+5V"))
 (segment (start 160 84) (end 175.655 84) (width 0.2) (layer "B.Cu") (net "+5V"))
 (segment (start 139 84.5) (end 140.17 85.67) (width 0.2) (layer "B.Cu") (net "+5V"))
 (segment (start 139 82.5) (end 139 84.5) (width 0.2) (layer "B.Cu") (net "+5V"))
 (segment (start 175.655 84) (end 176.655 85) (width 0.2) (layer "B.Cu") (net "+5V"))
 (segment (start 187.74 73.26) (end 190.76 73.26) (width 0.2) (layer "B.Cu") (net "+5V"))
 (segment (start 141.775 85.395) (end 141.5 85.67) (width 0.2) (layer "B.Cu") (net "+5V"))
 (segment (start 141.5 85.67) (end 141.655 85.67) (width 0.2) (layer "B.Cu") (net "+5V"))
 (segment (start 140 81.5) (end 139 82.5) (width 0.2) (layer "B.Cu") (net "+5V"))
 (segment (start 176.655 84.345) (end 187.74 73.26) (width 0.2) (layer "B.Cu") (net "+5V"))
 (segment (start 175.155 85.67) (end 176.655 87.17) (width 0.2) (layer "B.Cu") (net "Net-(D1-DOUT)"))
 (segment (start 164.88 85.67) (end 175.155 85.67) (width 0.2) (layer "B.Cu") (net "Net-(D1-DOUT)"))
 (segment (start 147.225 85.25) (end 147.225 85.395) (width 0.2) (layer "B.Cu") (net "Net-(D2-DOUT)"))
 (segment (start 147.225 85.395) (end 147.5 85.67) (width 0.2) (layer "B.Cu") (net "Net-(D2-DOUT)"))
 (segment (start 157.93 85.67) (end 159.43 87.17) (width 0.2) (layer "B.Cu") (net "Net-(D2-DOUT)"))
 (segment (start 147.5 85.67) (end 157.93 85.67) (width 0.2) (layer "B.Cu") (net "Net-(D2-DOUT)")))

